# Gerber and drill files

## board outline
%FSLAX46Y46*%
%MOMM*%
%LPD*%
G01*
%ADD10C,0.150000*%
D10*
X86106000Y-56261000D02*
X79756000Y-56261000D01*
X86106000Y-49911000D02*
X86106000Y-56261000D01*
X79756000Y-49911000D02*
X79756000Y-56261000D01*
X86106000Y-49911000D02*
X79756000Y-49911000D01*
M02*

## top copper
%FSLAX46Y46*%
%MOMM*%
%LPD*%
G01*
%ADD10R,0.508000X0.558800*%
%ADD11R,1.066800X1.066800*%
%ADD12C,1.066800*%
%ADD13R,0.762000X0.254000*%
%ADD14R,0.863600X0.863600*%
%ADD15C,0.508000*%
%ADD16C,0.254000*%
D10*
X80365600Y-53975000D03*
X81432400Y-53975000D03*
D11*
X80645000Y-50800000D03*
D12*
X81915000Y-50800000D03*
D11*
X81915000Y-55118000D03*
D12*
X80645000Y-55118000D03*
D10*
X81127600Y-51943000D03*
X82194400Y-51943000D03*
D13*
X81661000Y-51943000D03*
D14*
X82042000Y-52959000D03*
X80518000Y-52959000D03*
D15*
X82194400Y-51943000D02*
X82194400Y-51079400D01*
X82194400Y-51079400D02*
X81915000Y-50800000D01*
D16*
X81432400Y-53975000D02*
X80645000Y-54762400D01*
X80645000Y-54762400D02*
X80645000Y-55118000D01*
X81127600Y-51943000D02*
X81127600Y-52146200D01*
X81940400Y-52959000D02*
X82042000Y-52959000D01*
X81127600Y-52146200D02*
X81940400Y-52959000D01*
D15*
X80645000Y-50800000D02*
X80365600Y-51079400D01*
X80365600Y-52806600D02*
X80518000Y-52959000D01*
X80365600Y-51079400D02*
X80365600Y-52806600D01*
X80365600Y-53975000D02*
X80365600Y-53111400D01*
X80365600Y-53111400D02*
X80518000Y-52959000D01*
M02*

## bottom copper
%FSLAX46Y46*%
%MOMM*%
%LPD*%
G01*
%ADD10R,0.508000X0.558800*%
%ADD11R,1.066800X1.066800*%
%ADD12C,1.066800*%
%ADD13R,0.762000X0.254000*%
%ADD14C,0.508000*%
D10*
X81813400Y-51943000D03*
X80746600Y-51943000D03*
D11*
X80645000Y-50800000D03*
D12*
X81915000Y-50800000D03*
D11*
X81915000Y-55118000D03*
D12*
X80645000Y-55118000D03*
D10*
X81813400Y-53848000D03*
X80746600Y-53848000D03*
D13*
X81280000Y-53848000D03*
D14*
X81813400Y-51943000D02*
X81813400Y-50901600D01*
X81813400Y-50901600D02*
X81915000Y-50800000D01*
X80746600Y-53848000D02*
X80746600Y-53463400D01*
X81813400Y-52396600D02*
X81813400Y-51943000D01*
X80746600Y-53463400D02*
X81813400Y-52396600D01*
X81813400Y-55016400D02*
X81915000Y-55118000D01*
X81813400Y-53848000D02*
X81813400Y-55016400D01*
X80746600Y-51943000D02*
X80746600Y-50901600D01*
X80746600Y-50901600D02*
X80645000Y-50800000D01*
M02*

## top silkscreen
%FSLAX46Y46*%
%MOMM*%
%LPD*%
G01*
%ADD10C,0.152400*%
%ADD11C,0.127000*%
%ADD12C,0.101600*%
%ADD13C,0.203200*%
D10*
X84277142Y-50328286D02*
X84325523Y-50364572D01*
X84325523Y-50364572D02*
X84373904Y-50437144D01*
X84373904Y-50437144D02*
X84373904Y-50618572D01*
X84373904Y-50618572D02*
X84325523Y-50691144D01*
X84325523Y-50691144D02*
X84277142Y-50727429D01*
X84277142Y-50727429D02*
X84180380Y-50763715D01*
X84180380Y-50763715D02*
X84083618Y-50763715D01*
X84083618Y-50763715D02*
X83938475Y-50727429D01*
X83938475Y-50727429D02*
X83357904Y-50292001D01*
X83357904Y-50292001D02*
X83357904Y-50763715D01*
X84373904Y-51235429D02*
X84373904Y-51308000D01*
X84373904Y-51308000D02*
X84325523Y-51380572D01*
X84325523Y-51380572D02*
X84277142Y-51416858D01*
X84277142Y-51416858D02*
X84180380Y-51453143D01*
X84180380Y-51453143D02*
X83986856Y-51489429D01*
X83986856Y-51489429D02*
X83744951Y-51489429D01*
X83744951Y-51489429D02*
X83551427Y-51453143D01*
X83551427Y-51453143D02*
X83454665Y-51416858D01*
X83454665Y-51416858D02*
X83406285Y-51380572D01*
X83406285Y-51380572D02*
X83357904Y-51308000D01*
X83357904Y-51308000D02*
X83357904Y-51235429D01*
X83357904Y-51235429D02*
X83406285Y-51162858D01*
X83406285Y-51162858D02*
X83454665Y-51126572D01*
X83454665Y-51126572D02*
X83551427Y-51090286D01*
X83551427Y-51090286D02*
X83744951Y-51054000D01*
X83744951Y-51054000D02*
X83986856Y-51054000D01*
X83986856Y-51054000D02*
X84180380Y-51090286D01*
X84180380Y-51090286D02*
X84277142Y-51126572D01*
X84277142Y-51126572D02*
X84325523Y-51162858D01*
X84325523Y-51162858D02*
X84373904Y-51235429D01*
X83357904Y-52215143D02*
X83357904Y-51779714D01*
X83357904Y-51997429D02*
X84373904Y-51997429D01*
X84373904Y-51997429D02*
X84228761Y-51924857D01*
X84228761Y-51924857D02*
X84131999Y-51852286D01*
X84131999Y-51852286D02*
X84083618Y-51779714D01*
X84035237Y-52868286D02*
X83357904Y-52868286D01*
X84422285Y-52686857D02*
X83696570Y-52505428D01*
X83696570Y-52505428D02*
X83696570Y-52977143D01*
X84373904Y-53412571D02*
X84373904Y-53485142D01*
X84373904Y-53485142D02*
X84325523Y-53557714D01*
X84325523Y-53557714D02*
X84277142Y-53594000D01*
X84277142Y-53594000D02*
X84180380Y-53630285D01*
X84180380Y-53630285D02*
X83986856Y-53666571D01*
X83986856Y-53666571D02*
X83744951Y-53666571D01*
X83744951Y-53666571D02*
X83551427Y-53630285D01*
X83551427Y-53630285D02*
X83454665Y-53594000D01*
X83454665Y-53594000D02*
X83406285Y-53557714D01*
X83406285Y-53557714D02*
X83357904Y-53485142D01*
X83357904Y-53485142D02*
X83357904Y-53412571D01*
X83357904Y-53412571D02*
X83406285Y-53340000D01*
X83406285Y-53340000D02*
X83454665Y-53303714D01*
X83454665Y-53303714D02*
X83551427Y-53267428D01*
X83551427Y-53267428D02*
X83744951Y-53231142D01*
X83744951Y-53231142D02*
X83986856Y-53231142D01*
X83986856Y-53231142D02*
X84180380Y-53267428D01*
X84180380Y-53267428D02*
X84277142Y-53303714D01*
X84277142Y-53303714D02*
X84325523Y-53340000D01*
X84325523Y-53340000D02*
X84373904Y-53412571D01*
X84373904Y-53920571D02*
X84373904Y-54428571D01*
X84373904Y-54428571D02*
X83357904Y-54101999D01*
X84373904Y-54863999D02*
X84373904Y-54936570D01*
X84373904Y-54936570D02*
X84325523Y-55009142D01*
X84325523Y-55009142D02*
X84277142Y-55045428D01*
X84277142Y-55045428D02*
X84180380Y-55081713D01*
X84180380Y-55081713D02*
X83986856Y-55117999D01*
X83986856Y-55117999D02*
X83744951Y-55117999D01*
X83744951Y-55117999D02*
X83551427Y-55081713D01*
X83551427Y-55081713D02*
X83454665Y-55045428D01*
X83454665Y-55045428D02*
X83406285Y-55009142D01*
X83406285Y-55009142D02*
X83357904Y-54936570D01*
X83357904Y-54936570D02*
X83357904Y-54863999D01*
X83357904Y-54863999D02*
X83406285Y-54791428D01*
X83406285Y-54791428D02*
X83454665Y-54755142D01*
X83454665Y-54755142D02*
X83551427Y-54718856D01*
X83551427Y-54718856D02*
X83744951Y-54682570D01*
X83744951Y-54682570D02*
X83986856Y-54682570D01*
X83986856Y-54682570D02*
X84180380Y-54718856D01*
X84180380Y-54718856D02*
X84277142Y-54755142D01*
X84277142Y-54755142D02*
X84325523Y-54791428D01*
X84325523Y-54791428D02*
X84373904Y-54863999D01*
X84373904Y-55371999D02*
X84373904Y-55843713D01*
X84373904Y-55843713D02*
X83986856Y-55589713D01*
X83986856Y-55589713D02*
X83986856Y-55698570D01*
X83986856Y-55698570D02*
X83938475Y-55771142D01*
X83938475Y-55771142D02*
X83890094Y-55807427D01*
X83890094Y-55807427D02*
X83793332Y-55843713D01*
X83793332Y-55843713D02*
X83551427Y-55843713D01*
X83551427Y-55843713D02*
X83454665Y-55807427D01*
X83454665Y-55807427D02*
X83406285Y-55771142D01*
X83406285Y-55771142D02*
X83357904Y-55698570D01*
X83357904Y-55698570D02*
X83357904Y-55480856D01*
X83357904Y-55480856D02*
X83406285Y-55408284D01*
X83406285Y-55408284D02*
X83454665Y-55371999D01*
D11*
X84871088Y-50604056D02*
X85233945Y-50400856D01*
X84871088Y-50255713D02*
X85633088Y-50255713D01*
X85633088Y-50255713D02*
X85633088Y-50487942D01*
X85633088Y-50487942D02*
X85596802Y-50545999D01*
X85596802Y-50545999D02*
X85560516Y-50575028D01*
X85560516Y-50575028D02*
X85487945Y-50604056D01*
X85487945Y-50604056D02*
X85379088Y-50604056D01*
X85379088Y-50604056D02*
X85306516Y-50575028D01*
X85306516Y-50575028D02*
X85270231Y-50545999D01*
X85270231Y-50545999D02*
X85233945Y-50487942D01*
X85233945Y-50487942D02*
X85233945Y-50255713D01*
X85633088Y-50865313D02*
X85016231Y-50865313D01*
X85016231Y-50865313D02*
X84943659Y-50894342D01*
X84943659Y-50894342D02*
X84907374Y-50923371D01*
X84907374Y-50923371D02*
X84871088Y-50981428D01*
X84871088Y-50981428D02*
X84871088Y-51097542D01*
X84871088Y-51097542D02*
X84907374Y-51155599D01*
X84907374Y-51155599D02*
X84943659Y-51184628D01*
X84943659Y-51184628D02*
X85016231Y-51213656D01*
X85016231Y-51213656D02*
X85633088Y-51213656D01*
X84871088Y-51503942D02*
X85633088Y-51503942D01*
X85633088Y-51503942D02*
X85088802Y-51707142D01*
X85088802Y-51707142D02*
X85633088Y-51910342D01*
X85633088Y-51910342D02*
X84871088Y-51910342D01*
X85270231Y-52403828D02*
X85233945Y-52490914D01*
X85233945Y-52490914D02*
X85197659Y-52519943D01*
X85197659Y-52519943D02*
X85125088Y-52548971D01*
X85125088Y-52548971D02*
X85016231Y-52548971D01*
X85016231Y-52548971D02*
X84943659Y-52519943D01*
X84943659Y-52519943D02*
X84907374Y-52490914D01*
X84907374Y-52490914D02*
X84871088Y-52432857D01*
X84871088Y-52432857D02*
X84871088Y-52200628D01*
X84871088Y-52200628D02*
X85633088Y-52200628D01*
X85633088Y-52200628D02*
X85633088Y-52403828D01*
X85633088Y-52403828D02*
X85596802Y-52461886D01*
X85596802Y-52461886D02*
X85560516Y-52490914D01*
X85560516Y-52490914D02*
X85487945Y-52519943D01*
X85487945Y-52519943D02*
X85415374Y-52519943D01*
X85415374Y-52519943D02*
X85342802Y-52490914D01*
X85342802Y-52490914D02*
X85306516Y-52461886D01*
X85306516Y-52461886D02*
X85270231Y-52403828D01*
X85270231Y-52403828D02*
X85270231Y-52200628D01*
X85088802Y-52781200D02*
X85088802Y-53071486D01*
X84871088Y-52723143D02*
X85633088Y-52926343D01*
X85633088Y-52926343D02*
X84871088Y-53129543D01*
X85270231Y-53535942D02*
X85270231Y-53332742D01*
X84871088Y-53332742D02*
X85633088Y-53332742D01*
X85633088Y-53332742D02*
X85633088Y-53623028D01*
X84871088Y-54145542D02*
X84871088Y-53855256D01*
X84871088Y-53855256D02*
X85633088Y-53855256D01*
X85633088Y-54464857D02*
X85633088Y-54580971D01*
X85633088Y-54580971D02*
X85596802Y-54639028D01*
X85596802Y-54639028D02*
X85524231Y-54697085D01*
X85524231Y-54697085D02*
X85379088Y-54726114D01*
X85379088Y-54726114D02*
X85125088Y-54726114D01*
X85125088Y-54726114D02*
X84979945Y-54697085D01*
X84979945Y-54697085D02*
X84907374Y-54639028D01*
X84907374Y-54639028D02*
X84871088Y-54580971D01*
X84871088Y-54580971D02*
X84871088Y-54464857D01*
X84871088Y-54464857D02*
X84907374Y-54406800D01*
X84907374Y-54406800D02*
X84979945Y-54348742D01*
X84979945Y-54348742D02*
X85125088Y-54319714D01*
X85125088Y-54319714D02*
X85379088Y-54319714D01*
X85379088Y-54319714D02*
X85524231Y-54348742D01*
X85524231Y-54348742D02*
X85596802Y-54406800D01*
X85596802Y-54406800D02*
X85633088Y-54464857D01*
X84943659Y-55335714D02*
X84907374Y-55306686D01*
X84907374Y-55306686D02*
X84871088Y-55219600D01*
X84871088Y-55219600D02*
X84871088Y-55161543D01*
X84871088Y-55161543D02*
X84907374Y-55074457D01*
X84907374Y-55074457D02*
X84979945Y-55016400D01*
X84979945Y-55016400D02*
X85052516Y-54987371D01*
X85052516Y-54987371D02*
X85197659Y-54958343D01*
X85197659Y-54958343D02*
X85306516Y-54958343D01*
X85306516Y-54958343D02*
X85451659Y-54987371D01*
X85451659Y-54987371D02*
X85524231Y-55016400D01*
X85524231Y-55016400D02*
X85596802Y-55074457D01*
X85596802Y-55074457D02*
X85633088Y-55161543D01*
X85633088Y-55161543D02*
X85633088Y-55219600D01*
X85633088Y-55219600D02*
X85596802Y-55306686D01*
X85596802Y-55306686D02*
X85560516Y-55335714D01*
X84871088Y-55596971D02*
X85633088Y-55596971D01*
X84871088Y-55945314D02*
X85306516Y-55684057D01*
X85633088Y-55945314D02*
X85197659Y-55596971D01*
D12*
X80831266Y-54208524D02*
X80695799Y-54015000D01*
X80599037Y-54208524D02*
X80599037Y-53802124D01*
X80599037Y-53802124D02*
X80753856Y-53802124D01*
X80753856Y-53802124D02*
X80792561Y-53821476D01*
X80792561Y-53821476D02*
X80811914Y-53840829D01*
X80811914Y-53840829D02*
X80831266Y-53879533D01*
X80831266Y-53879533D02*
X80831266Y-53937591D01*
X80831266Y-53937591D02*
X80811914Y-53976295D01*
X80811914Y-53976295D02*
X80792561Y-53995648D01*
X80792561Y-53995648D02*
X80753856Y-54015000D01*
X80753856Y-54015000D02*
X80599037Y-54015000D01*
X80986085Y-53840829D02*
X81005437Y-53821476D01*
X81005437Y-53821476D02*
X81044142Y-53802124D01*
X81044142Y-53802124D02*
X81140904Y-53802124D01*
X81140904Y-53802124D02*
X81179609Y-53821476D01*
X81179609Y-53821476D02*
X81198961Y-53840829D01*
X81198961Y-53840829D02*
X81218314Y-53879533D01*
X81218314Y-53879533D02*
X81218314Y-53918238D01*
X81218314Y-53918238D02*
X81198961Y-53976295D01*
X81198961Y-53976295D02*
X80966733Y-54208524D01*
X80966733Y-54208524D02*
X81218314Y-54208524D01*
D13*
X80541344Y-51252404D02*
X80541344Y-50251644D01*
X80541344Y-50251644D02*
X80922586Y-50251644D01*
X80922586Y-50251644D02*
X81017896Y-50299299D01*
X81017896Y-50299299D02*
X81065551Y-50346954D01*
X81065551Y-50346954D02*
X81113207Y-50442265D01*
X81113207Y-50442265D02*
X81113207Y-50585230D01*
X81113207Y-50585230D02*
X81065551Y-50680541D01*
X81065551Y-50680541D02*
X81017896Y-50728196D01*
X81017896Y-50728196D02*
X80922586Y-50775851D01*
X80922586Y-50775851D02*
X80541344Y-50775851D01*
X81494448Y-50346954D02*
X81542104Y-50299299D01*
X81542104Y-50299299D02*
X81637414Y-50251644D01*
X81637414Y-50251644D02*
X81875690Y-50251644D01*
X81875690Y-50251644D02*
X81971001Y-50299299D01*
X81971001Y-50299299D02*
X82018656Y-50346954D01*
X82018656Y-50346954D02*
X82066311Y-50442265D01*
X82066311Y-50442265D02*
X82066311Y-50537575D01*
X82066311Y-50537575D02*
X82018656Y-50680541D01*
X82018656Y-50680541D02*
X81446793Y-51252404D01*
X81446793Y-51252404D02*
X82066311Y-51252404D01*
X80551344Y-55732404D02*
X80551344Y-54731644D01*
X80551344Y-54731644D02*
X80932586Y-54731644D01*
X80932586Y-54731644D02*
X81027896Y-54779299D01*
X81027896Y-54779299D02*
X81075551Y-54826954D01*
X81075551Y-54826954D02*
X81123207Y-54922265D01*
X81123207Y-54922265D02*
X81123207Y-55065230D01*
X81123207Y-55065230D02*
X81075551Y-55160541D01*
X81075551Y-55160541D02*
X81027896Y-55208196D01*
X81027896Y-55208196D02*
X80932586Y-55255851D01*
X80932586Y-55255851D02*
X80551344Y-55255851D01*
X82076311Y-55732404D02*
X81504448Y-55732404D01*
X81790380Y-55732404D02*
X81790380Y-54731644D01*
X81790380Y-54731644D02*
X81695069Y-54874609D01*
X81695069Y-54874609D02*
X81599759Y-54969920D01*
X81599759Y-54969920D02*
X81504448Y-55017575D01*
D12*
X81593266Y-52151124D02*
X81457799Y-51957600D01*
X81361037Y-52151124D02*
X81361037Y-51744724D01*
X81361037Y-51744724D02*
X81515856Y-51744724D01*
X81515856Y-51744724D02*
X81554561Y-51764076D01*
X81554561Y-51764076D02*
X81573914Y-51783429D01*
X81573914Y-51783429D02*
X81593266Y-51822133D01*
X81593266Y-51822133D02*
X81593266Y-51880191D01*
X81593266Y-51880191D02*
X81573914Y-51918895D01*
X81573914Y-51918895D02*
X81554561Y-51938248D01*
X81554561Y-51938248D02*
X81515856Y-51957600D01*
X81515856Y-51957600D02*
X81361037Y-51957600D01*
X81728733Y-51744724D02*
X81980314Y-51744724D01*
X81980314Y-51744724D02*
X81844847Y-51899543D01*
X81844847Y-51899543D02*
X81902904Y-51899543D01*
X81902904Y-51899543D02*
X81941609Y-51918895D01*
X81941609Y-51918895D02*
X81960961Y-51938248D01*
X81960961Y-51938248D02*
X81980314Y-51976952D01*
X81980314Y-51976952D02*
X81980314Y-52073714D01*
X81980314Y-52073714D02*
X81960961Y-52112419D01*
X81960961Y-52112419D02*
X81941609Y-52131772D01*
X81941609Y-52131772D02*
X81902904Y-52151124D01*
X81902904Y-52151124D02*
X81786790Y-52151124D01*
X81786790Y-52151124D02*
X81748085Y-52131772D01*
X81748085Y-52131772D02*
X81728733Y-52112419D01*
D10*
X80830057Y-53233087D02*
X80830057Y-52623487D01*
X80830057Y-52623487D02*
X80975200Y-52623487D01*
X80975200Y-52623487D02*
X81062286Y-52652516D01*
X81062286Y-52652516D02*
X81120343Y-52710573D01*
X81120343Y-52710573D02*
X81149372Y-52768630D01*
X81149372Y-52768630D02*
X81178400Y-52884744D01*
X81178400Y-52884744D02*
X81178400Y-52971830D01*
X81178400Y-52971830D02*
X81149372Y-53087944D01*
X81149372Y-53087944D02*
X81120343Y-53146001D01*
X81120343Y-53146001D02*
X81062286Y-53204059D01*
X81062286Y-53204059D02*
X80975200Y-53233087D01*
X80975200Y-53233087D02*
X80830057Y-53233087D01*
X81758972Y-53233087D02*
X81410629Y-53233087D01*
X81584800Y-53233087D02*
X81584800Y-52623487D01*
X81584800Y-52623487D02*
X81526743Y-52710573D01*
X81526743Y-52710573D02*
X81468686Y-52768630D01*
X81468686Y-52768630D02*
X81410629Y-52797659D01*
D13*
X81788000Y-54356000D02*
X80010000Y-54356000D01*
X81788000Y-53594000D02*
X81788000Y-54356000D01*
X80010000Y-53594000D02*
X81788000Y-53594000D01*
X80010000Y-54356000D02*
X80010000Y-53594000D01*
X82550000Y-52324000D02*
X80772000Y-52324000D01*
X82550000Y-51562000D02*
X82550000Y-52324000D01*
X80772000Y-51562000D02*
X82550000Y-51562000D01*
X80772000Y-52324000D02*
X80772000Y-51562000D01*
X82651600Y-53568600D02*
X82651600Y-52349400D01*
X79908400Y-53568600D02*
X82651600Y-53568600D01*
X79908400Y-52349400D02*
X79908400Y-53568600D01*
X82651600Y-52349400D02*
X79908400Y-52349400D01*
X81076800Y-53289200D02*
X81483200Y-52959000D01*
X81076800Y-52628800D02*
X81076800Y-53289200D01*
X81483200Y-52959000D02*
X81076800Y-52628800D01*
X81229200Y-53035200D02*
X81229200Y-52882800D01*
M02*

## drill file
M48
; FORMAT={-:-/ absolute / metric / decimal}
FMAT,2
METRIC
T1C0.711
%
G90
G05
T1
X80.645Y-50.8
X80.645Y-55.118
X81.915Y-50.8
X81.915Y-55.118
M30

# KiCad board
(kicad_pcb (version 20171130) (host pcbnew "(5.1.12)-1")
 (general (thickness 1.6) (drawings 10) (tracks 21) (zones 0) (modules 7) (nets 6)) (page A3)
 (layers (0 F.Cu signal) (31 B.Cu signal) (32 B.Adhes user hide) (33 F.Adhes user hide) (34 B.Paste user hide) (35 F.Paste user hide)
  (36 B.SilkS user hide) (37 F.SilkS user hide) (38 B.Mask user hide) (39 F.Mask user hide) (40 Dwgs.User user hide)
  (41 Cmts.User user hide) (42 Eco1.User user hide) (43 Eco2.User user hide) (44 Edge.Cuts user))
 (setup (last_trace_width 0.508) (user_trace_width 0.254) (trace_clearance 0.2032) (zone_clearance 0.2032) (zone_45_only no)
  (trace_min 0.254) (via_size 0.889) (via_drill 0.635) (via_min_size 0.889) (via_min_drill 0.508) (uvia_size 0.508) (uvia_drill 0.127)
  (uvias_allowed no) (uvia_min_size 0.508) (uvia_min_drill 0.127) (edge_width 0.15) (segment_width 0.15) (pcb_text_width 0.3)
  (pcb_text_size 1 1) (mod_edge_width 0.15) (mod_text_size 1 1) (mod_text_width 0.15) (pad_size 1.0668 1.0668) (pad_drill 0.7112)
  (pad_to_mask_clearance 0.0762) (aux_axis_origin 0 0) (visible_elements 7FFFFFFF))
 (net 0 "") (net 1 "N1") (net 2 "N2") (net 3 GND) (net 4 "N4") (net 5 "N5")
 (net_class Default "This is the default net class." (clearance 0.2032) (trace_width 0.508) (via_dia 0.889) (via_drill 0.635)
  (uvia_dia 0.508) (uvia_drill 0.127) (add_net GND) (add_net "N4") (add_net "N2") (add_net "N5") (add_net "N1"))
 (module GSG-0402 (layer F.Cu) (at 80.899 53.975 180) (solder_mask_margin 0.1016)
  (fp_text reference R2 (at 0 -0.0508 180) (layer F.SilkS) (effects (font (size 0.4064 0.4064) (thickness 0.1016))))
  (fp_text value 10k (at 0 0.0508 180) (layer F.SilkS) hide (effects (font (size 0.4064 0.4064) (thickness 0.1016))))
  (fp_line (start -0.889 -0.381) (end 0.889 -0.381) (layer F.SilkS) (width 0.2032))
  (fp_line (start -0.889 0.381) (end -0.889 -0.381) (layer F.SilkS) (width 0.2032))
  (fp_line (start 0.889 0.381) (end -0.889 0.381) (layer F.SilkS) (width 0.2032))
  (fp_line (start 0.889 -0.381) (end 0.889 0.381) (layer F.SilkS) (width 0.2032))
  (pad 2 smd rect (at 0.5334 0 180) (size 0.508 0.5588) (layers F.Cu F.Paste F.Mask) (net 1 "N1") (solder_mask_margin 0.1016))
  (pad 1 smd rect (at -0.5334 0 180) (size 0.508 0.5588) (layers F.Cu F.Paste F.Mask) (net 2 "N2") (die_length -1518.485687)
   (solder_mask_margin 0.1016)))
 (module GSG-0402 (layer B.Cu) (at 81.28 51.943) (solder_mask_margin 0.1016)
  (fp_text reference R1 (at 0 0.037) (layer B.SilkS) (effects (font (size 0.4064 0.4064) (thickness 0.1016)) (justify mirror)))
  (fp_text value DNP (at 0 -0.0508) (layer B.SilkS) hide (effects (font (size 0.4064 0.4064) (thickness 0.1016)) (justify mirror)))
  (pad 2 smd rect (at 0.5334 0) (size 0.508 0.5588) (layers B.Cu B.Paste B.Mask) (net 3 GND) (solder_mask_margin 0.1016))
  (pad 1 smd rect (at -0.5334 0) (size 0.508 0.5588) (layers B.Cu B.Paste B.Mask) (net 1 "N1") (die_length -1518.485687)
   (solder_mask_margin 0.1016)))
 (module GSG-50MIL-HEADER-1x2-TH (layer F.Cu) (at 81.28 50.8)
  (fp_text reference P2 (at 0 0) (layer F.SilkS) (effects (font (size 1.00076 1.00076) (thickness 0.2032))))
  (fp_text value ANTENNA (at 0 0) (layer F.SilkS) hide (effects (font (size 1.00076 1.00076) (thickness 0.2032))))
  (pad 1 thru_hole rect (at -0.635 0) (size 1.0668 1.0668) (drill 0.7112) (layers *.Cu *.Mask) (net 1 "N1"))
  (pad 2 thru_hole circle (at 0.635 0) (size 1.0668 1.0668) (drill 0.7112) (layers *.Cu *.Mask) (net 3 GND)))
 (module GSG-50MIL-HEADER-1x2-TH (layer F.Cu) (at 81.28 55.118 180)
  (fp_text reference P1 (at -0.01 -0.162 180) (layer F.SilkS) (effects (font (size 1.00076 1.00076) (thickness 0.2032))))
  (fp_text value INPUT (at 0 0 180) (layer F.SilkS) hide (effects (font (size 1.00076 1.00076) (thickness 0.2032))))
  (pad 1 thru_hole rect (at -0.635 0 180) (size 1.0668 1.0668) (drill 0.7112) (layers *.Cu *.Mask) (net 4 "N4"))
  (pad 2 thru_hole circle (at 0.635 0 180) (size 1.0668 1.0668) (drill 0.7112) (layers *.Cu *.Mask) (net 2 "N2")))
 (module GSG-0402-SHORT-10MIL (layer B.Cu) (at 81.28 53.848) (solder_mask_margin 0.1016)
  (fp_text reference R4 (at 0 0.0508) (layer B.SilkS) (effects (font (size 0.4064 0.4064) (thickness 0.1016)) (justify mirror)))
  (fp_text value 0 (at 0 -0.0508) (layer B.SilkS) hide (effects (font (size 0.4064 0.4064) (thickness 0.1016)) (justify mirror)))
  (pad 2 smd rect (at 0.5334 0) (size 0.508 0.5588) (layers B.Cu B.Mask) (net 4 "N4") (solder_mask_margin 0.1016))
  (pad 1 smd rect (at -0.5334 0) (size 0.508 0.5588) (layers B.Cu B.Mask) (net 3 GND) (die_length -1518.485687) (solder_mask_margin 0.1016))
  (pad "" smd rect (at 0 0) (size 0.762 0.254) (layers B.Cu B.Mask)))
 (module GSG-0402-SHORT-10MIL (layer F.Cu) (at 81.661 51.943 180) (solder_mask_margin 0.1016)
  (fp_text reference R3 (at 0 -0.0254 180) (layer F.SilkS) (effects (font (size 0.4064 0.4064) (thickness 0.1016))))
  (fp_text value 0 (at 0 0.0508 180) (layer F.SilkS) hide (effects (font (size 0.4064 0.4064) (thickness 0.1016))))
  (fp_line (start -0.889 -0.381) (end 0.889 -0.381) (layer F.SilkS) (width 0.2032))
  (fp_line (start -0.889 0.381) (end -0.889 -0.381) (layer F.SilkS) (width 0.2032))
  (fp_line (start 0.889 0.381) (end -0.889 0.381) (layer F.SilkS) (width 0.2032))
  (fp_line (start 0.889 -0.381) (end 0.889 0.381) (layer F.SilkS) (width 0.2032))
  (pad 2 smd rect (at 0.5334 0 180) (size 0.508 0.5588) (layers F.Cu F.Mask) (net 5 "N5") (solder_mask_margin 0.1016))
  (pad 1 smd rect (at -0.5334 0 180) (size 0.508 0.5588) (layers F.Cu F.Mask) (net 3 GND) (die_length -1518.485687)
   (solder_mask_margin 0.1016))
  (pad "" smd rect (at 0 0 180) (size 0.762 0.254) (layers F.Cu F.Mask)))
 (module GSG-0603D (layer F.Cu) (at 81.28 52.959) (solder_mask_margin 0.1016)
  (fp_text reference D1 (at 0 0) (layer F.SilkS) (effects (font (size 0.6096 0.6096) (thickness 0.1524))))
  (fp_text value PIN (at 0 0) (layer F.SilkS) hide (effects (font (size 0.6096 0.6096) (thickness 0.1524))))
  (fp_line (start 1.3716 0.6096) (end 1.3716 -0.6096) (layer F.SilkS) (width 0.2032))
  (fp_line (start -1.3716 0.6096) (end 1.3716 0.6096) (layer F.SilkS) (width 0.2032))
  (fp_line (start -1.3716 -0.6096) (end -1.3716 0.6096) (layer F.SilkS) (width 0.2032))
  (fp_line (start 1.3716 -0.6096) (end -1.3716 -0.6096) (layer F.SilkS) (width 0.2032))
  (fp_line (start -0.2032 0.3302) (end 0.2032 0) (layer F.SilkS) (width 0.2032))
  (fp_line (start -0.2032 -0.3302) (end -0.2032 0.3302) (layer F.SilkS) (width 0.2032))
  (fp_line (start 0.2032 0) (end -0.2032 -0.3302) (layer F.SilkS) (width 0.2032))
  (fp_line (start -0.0508 0.0762) (end -0.0508 -0.0762) (layer F.SilkS) (width 0.2032))
  (pad 2 smd rect (at 0.762 0) (size 0.8636 0.8636) (layers F.Cu F.Paste F.Mask) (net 5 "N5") (die_length 0.04572)
   (solder_mask_margin 0.1016) (clearance 0.1778))
  (pad 1 smd rect (at -0.762 0) (size 0.8636 0.8636) (layers F.Cu F.Paste F.Mask) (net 1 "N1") (die_length 0.08382)
   (solder_mask_margin 0.1016) (clearance 0.1778)))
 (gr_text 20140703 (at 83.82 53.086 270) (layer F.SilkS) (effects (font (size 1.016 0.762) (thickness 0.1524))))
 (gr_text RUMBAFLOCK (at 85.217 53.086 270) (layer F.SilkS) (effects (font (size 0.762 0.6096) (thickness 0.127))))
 (gr_line (start 86.106 56.261) (end 79.756 56.261) (angle 90) (layer Edge.Cuts) (width 0.15))
 (gr_line (start 86.106 49.911) (end 86.106 56.261) (angle 90) (layer Edge.Cuts) (width 0.15))
 (gr_line (start 79.756 49.911) (end 79.756 56.261) (angle 90) (layer Edge.Cuts) (width 0.15))
 (gr_line (start 86.106 49.911) (end 79.756 49.911) (angle 90) (layer Edge.Cuts) (width 0.15))
 (segment (start 82.1944 51.943) (end 82.1944 51.0794) (width 0.508) (layer F.Cu) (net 3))
 (segment (start 82.1944 51.0794) (end 81.915 50.8) (width 0.508) (layer F.Cu) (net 3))
 (segment (start 81.8134 51.943) (end 81.8134 50.9016) (width 0.508) (layer B.Cu) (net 3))
 (segment (start 81.8134 50.9016) (end 81.915 50.8) (width 0.508) (layer B.Cu) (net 3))
 (segment (start 80.7466 53.848) (end 80.7466 53.4634) (width 0.508) (layer B.Cu) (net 3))
 (segment (start 81.8134 52.3966) (end 81.8134 51.943) (width 0.508) (layer B.Cu) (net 3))
 (segment (start 80.7466 53.4634) (end 81.8134 52.3966) (width 0.508) (layer B.Cu) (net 3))
 (segment (start 81.8134 55.0164) (end 81.915 55.118) (width 0.508) (layer B.Cu) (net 4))
 (segment (start 81.8134 53.848) (end 81.8134 55.0164) (width 0.508) (layer B.Cu) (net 4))
 (segment (start 81.4324 53.975) (end 80.645 54.7624) (width 0.254) (layer F.Cu) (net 2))
 (segment (start 80.645 54.7624) (end 80.645 55.118) (width 0.254) (layer F.Cu) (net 2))
 (segment (start 81.1276 51.943) (end 81.1276 52.1462) (width 0.254) (layer F.Cu) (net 5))
 (segment (start 81.9404 52.959) (end 82.042 52.959) (width 0.254) (layer F.Cu) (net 5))
 (segment (start 81.1276 52.1462) (end 81.9404 52.959) (width 0.254) (layer F.Cu) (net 5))
 (segment (start 80.645 50.8) (end 80.3656 51.0794) (width 0.508) (layer F.Cu) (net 1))
 (segment (start 80.3656 52.8066) (end 80.518 52.959) (width 0.508) (layer F.Cu) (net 1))
 (segment (start 80.3656 51.0794) (end 80.3656 52.8066) (width 0.508) (layer F.Cu) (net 1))
 (segment (start 80.3656 53.975) (end 80.3656 53.1114) (width 0.508) (layer F.Cu) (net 1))
 (segment (start 80.3656 53.1114) (end 80.518 52.959) (width 0.508) (layer F.Cu) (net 1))
 (segment (start 80.7466 51.943) (end 80.7466 50.9016) (width 0.508) (layer B.Cu) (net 1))
 (segment (start 80.7466 50.9016) (end 80.645 50.8) (width 0.508) (layer B.Cu) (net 1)))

